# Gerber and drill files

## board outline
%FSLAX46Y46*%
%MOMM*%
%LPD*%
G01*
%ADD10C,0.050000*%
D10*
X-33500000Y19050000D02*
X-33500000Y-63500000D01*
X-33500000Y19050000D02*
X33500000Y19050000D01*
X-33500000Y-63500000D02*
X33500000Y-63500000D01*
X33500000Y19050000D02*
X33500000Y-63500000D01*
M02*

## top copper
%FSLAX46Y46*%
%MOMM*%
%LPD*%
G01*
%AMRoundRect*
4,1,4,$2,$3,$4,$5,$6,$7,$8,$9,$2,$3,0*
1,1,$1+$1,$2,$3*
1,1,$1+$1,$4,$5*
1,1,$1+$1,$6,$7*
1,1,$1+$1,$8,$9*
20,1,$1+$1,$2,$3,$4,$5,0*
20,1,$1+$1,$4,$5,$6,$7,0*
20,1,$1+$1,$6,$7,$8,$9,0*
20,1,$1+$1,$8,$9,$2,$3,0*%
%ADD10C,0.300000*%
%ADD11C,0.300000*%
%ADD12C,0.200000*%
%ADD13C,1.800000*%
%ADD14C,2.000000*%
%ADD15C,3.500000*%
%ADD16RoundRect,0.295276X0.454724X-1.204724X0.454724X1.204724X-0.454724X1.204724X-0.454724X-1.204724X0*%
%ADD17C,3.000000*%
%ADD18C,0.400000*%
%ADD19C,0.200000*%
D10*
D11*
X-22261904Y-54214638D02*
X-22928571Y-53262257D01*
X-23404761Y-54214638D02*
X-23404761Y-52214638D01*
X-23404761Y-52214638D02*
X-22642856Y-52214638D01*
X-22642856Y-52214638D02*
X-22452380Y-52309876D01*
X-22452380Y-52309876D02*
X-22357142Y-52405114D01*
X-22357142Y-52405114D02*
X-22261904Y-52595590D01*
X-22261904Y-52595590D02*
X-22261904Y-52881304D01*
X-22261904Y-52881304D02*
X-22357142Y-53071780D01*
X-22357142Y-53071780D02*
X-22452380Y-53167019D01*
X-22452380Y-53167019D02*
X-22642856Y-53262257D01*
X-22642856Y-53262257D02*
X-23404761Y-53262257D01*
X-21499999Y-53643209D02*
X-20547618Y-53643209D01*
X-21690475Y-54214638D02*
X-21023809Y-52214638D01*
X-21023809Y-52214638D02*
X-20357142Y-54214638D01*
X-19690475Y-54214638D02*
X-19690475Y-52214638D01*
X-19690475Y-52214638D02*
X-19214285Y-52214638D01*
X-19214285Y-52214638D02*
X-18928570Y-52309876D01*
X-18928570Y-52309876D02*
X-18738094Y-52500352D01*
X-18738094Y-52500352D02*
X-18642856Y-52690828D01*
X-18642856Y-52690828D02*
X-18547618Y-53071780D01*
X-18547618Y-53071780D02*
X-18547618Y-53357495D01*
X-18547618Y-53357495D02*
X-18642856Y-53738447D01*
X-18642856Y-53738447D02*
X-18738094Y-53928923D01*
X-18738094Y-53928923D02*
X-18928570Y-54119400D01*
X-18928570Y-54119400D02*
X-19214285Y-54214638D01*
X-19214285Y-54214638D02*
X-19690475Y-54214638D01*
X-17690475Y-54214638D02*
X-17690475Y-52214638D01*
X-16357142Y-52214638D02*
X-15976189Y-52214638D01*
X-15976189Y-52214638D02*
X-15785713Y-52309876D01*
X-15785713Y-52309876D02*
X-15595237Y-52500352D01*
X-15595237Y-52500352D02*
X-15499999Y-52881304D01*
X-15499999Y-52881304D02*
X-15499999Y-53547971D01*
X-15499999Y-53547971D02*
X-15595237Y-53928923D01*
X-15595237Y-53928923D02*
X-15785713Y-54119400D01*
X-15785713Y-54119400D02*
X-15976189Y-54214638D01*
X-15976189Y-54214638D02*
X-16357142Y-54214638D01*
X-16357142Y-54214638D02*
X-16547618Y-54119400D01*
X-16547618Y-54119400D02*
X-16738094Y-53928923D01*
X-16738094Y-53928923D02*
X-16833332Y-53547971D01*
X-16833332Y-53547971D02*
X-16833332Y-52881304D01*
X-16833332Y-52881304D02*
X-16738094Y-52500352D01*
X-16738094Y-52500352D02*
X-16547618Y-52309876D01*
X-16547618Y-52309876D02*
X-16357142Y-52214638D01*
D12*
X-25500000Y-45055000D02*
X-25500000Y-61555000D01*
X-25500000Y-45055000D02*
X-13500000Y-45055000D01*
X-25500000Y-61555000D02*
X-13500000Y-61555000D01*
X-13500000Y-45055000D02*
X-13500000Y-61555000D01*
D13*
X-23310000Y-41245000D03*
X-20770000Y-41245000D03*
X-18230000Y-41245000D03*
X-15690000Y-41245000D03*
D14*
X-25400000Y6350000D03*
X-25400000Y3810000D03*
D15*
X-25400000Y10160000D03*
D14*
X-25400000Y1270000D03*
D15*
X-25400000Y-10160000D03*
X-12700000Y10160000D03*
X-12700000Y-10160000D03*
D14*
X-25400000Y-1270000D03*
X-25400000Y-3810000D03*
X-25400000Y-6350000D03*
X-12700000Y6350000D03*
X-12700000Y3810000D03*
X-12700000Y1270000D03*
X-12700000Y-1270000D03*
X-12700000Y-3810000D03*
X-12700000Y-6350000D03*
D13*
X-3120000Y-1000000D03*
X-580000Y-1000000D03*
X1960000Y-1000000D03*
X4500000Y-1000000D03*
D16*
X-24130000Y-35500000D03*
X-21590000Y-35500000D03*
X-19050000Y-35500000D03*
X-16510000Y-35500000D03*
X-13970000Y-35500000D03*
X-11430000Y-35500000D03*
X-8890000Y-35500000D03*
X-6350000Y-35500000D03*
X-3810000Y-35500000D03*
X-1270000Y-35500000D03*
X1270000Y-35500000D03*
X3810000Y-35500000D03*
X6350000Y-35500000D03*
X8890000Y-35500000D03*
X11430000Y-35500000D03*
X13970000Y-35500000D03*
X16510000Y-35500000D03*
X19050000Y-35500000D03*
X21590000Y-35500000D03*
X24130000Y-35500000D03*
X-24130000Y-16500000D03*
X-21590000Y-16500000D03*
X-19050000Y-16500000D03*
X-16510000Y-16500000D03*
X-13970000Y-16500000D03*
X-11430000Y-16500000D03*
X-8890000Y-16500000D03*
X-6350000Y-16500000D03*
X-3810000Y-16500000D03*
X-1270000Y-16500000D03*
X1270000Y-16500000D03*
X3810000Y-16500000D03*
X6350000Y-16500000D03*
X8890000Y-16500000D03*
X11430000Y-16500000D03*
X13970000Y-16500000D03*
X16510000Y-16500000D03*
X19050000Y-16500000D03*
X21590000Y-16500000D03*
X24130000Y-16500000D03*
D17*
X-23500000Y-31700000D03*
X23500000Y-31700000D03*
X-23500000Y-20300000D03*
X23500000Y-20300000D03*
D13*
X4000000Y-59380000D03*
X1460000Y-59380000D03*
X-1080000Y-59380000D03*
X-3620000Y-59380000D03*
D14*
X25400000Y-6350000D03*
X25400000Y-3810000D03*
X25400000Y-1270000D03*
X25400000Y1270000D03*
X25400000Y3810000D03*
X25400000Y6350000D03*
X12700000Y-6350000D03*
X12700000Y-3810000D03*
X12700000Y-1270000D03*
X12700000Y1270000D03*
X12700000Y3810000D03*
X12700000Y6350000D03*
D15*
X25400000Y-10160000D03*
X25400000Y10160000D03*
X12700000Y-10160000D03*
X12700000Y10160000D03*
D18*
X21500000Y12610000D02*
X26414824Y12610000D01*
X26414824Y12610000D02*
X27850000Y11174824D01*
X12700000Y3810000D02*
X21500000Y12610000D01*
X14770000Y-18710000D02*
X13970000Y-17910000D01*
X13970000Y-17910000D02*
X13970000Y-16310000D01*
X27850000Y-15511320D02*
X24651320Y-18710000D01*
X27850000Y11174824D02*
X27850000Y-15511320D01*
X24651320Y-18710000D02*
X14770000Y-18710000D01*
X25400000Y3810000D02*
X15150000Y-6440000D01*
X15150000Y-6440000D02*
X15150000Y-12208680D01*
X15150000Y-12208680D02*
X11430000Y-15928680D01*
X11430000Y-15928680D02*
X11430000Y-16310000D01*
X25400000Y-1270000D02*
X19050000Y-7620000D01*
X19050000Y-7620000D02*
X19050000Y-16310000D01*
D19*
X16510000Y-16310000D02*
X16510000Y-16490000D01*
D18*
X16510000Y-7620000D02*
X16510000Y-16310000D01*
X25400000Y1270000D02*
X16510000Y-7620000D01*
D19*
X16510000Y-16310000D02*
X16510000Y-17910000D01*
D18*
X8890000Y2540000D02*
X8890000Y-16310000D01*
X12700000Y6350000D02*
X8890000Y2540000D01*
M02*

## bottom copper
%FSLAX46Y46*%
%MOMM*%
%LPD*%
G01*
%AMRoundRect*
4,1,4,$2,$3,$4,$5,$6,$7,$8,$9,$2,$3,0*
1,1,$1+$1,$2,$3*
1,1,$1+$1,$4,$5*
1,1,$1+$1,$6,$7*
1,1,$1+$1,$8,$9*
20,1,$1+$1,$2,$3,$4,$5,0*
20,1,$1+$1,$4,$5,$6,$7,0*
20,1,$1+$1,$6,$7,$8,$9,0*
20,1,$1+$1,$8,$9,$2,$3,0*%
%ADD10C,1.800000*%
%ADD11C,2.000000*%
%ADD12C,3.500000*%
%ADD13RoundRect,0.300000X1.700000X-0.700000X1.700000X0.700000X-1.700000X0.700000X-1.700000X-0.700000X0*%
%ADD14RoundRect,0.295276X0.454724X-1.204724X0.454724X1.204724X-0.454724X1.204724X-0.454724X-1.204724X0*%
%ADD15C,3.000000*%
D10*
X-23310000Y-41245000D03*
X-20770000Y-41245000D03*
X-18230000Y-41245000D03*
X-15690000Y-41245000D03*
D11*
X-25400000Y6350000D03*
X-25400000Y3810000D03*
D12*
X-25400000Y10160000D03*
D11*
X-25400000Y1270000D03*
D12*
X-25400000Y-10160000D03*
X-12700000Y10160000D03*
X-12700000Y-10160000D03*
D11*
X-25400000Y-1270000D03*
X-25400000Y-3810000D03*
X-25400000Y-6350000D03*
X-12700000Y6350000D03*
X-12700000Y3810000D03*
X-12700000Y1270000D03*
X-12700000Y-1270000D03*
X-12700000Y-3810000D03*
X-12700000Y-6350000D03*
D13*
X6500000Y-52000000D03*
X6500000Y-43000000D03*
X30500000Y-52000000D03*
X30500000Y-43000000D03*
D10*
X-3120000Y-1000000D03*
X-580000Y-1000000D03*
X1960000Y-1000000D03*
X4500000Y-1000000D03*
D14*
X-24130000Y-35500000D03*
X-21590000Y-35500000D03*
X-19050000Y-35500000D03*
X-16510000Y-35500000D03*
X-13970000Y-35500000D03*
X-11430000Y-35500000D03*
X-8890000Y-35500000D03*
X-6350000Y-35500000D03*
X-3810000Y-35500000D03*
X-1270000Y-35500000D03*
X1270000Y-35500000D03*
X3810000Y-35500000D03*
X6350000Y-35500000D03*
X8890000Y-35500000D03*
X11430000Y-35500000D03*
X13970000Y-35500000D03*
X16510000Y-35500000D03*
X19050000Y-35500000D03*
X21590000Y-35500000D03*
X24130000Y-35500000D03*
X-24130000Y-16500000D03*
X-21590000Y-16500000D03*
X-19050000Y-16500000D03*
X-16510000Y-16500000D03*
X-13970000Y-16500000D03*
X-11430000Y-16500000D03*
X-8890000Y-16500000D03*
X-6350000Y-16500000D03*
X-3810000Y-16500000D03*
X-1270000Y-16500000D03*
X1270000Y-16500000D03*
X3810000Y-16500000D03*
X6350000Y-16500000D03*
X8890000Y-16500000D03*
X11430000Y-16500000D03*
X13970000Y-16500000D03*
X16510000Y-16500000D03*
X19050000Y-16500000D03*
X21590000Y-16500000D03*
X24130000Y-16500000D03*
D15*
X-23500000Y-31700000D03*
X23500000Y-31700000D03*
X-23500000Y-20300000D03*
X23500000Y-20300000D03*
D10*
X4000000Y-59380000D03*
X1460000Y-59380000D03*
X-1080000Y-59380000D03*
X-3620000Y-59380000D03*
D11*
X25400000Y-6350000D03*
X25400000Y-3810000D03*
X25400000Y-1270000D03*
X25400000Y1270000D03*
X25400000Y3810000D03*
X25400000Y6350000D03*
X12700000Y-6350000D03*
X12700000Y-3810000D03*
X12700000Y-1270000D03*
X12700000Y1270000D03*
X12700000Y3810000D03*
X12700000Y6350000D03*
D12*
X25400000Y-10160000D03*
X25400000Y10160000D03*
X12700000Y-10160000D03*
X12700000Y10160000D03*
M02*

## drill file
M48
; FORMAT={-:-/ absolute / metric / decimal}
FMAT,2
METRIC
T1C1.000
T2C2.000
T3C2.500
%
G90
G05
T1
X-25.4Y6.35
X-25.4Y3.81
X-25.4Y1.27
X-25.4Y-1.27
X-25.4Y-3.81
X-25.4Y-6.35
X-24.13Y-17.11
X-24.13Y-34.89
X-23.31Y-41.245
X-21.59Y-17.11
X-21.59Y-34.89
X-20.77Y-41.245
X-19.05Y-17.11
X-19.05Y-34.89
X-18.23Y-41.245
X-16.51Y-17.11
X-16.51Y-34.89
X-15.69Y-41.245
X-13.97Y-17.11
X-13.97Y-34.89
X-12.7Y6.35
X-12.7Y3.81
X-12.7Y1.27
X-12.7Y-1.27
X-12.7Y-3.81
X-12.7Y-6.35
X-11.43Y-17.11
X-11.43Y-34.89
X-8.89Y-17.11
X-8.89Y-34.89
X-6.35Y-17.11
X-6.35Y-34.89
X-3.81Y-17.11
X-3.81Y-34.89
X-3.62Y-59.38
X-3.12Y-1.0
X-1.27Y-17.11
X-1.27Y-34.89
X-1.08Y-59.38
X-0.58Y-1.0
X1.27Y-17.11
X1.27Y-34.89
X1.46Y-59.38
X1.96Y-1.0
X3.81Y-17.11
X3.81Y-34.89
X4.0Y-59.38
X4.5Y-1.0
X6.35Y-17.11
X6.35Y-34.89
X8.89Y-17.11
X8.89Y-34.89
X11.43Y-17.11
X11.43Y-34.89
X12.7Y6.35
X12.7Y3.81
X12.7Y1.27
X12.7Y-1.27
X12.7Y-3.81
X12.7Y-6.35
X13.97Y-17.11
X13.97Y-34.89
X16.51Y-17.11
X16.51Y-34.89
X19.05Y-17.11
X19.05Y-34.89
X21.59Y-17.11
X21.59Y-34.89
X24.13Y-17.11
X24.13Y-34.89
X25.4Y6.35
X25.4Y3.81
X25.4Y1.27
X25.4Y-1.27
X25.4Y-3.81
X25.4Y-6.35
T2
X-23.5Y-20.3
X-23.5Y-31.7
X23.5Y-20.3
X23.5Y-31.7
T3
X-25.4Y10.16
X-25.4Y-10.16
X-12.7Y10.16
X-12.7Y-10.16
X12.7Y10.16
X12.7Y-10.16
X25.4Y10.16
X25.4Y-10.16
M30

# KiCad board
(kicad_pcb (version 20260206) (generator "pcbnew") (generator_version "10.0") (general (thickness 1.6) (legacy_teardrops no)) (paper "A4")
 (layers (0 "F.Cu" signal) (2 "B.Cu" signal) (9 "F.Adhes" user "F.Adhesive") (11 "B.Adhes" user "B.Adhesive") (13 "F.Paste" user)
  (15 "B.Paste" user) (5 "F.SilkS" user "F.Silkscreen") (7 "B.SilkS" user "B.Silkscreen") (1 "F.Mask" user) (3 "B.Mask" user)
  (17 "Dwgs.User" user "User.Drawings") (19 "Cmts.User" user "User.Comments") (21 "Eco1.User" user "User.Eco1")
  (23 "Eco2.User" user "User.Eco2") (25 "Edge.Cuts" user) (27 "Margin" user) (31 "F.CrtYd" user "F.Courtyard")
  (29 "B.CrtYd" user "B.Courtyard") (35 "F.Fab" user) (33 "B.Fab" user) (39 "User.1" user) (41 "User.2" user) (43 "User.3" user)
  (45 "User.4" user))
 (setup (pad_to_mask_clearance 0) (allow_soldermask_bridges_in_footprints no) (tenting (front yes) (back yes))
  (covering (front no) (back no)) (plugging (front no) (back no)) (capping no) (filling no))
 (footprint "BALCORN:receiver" (layer "F.Cu") (at -19.5 53.305)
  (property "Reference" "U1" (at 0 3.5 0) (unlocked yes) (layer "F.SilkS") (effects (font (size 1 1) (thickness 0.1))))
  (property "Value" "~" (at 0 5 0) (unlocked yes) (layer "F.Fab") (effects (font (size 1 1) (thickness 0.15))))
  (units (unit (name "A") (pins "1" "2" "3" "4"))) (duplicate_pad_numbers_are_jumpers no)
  (fp_line (start -6 -8.25) (end -6 8.25) (stroke (width 0.2) (type default)) (layer "F.Cu"))
  (fp_line (start -6 -8.25) (end 6 -8.25) (stroke (width 0.2) (type default)) (layer "F.Cu"))
  (fp_line (start -6 8.25) (end 6 8.25) (stroke (width 0.2) (type default)) (layer "F.Cu"))
  (fp_line (start 6 -8.25) (end 6 8.25) (stroke (width 0.2) (type default)) (layer "F.Cu"))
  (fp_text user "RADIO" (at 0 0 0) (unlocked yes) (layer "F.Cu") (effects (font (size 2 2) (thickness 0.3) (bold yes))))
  (pad "1" thru_hole circle (at -3.81 -12.06) (size 1.8 1.8) (drill 1) (layers "*.Cu" "*.Mask") (remove_unused_layers no)
   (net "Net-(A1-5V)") (thermal_bridge_angle 90))
  (pad "2" thru_hole circle (at -1.27 -12.06) (size 1.8 1.8) (drill 1) (layers "*.Cu" "*.Mask") (remove_unused_layers no)
   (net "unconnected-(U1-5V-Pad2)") (thermal_bridge_angle 90))
  (pad "3" thru_hole circle (at 1.27 -12.06) (size 1.8 1.8) (drill 1) (layers "*.Cu" "*.Mask") (remove_unused_layers no)
   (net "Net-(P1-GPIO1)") (thermal_bridge_angle 90))
  (pad "4" thru_hole circle (at 3.81 -12.06) (size 1.8 1.8) (drill 1) (layers "*.Cu" "*.Mask") (remove_unused_layers no)
   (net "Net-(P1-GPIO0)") (thermal_bridge_angle 90)))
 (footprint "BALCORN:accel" (layer "F.Cu") (at -19.05 0)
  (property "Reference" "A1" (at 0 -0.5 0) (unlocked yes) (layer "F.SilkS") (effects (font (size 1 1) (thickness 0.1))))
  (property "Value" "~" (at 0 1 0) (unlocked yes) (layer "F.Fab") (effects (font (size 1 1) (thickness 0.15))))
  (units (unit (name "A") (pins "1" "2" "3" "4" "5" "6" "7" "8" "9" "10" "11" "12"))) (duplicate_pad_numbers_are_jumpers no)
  (pad "1" thru_hole circle (at -6.35 -6.35) (size 2 2) (drill 1) (layers "*.Cu" "*.Mask") (remove_unused_layers no) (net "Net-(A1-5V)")
   (thermal_bridge_angle 90))
  (pad "2" thru_hole circle (at -6.35 -3.81) (size 2 2) (drill 1) (layers "*.Cu" "*.Mask") (remove_unused_layers no)
   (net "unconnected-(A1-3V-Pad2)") (thermal_bridge_angle 90))
  (pad "3" thru_hole circle (at -6.35 -10.16) (size 3.5 3.5) (drill 2.5) (layers "*.Cu" "*.Mask") (remove_unused_layers no)
   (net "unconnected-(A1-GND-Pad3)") (thermal_bridge_angle 90))
  (pad "3" thru_hole circle (at -6.35 -1.27) (size 2 2) (drill 1) (layers "*.Cu" "*.Mask") (remove_unused_layers no)
   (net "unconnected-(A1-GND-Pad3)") (thermal_bridge_angle 90))
  (pad "3" thru_hole circle (at -6.35 10.16) (size 3.5 3.5) (drill 2.5) (layers "*.Cu" "*.Mask") (remove_unused_layers no)
   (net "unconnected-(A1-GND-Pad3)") (thermal_bridge_angle 90))
  (pad "3" thru_hole circle (at 6.35 -10.16) (size 3.5 3.5) (drill 2.5) (layers "*.Cu" "*.Mask") (remove_unused_layers no)
   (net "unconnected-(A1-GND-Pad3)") (thermal_bridge_angle 90))
  (pad "3" thru_hole circle (at 6.35 10.16) (size 3.5 3.5) (drill 2.5) (layers "*.Cu" "*.Mask") (remove_unused_layers no)
   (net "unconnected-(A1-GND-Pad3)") (thermal_bridge_angle 90))
  (pad "4" thru_hole circle (at -6.35 1.27) (size 2 2) (drill 1) (layers "*.Cu" "*.Mask") (remove_unused_layers no) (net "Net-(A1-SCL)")
   (thermal_bridge_angle 90))
  (pad "5" thru_hole circle (at -6.35 3.81) (size 2 2) (drill 1) (layers "*.Cu" "*.Mask") (remove_unused_layers no) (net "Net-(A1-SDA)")
   (thermal_bridge_angle 90))
  (pad "6" thru_hole circle (at -6.35 6.35) (size 2 2) (drill 1) (layers "*.Cu" "*.Mask") (remove_unused_layers no)
   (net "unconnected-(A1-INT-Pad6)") (thermal_bridge_angle 90))
  (pad "7" thru_hole circle (at 6.35 -6.35) (size 2 2) (drill 1) (layers "*.Cu" "*.Mask") (remove_unused_layers no)
   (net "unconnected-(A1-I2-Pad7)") (thermal_bridge_angle 90))
  (pad "8" thru_hole circle (at 6.35 -3.81) (size 2 2) (drill 1) (layers "*.Cu" "*.Mask") (remove_unused_layers no)
   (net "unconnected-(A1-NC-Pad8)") (thermal_bridge_angle 90))
  (pad "9" thru_hole circle (at 6.35 -1.27) (size 2 2) (drill 1) (layers "*.Cu" "*.Mask") (remove_unused_layers no)
   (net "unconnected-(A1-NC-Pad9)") (thermal_bridge_angle 90))
  (pad "10" thru_hole circle (at 6.35 1.27) (size 2 2) (drill 1) (layers "*.Cu" "*.Mask") (remove_unused_layers no)
   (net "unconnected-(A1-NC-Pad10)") (thermal_bridge_angle 90))
  (pad "11" thru_hole circle (at 6.35 3.81) (size 2 2) (drill 1) (layers "*.Cu" "*.Mask") (remove_unused_layers no) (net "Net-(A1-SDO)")
   (thermal_bridge_angle 90))
  (pad "12" thru_hole circle (at 6.35 6.35) (size 2 2) (drill 1) (layers "*.Cu" "*.Mask") (remove_unused_layers no) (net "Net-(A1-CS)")
   (thermal_bridge_angle 90)))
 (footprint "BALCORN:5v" (layer "F.Cu") (at 18.5 47.5 90)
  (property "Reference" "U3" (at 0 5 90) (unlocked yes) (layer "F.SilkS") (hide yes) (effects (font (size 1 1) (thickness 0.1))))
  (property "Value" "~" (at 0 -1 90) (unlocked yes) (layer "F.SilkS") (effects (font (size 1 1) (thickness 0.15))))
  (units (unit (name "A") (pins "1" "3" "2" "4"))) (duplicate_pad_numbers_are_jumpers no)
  (pad "1" smd roundrect (at -4.5 -12 90) (size 2 4) (layers "*.Mask" "B.Cu") (roundrect_rratio 0.15) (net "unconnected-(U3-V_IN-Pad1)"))
  (pad "2" smd roundrect (at 4.5 -12 90) (size 2 4) (layers "*.Mask" "B.Cu") (roundrect_rratio 0.15) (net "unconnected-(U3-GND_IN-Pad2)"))
  (pad "3" smd roundrect (at -4.5 12 90) (size 2 4) (layers "*.Mask" "B.Cu") (roundrect_rratio 0.15) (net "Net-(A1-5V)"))
  (pad "4" smd roundrect (at 4.5 12 90) (size 2 4) (layers "*.Mask" "B.Cu") (roundrect_rratio 0.15) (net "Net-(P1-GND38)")))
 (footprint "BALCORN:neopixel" (layer "F.Cu") (at 0.69 1)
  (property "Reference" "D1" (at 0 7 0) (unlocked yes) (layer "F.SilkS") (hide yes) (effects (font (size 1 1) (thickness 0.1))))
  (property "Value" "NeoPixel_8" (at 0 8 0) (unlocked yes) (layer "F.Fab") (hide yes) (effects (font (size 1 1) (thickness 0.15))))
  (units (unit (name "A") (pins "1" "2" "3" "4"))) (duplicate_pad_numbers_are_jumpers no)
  (pad "1" thru_hole circle (at -3.81 0) (size 1.8 1.8) (drill 1) (layers "*.Cu" "*.Mask") (remove_unused_layers no) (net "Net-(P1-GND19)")
   (thermal_bridge_angle 90))
  (pad "2" thru_hole circle (at -1.27 0) (size 1.8 1.8) (drill 1) (layers "*.Cu" "*.Mask") (remove_unused_layers no) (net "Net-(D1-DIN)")
   (thermal_bridge_angle 90))
  (pad "3" thru_hole circle (at 1.27 0) (size 1.8 1.8) (drill 1) (layers "*.Cu" "*.Mask") (remove_unused_layers no) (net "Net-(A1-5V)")
   (thermal_bridge_angle 90))
  (pad "4" thru_hole circle (at 3.81 0) (size 1.8 1.8) (drill 1) (layers "*.Cu" "*.Mask") (remove_unused_layers no) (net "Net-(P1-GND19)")
   (thermal_bridge_angle 90)))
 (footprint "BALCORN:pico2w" (layer "F.Cu") (at 0 26 90)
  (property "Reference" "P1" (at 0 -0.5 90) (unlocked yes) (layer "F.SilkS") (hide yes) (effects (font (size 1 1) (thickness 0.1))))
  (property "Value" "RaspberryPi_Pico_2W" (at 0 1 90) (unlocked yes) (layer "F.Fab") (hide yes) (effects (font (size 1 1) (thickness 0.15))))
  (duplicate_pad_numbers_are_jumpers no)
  (pad "1" thru_hole roundrect (at -8.89 -24.13 90) (size 3 1.5) (drill 1 (offset -0.61 0)) (layers "*.Cu" "*.Mask")
   (remove_unused_layers no) (roundrect_rratio 0.1968503937) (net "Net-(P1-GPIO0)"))
  (pad "2" thru_hole roundrect (at -8.89 -21.59 90) (size 3 1.5) (drill 1 (offset -0.61 0)) (layers "*.Cu" "*.Mask")
   (remove_unused_layers no) (roundrect_rratio 0.1968503937) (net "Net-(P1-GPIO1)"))
  (pad "3" thru_hole roundrect (at -8.89 -19.05 90) (size 3 1.5) (drill 1 (offset -0.61 0)) (layers "*.Cu" "*.Mask")
   (remove_unused_layers no) (roundrect_rratio 0.1968503937) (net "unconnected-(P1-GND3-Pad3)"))
  (pad "4" thru_hole roundrect (at -8.89 -16.51 90) (size 3 1.5) (drill 1 (offset -0.61 0)) (layers "*.Cu" "*.Mask")
   (remove_unused_layers no) (roundrect_rratio 0.1968503937) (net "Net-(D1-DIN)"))
  (pad "5" thru_hole roundrect (at -8.89 -13.97 90) (size 3 1.5) (drill 1 (offset -0.61 0)) (layers "*.Cu" "*.Mask")
   (remove_unused_layers no) (roundrect_rratio 0.1968503937) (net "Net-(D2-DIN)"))
  (pad "6" thru_hole roundrect (at -8.89 -11.43 90) (size 3 1.5) (drill 1 (offset -0.61 0)) (layers "*.Cu" "*.Mask")
   (remove_unused_layers no) (roundrect_rratio 0.1968503937) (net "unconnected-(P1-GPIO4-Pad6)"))
  (pad "7" thru_hole roundrect (at -8.89 -8.89 90) (size 3 1.5) (drill 1 (offset -0.61 0)) (layers "*.Cu" "*.Mask")
   (remove_unused_layers no) (roundrect_rratio 0.1968503937) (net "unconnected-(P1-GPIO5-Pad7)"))
  (pad "8" thru_hole roundrect (at -8.89 -6.35 90) (size 3 1.5) (drill 1 (offset -0.61 0)) (layers "*.Cu" "*.Mask")
   (remove_unused_layers no) (roundrect_rratio 0.1968503937) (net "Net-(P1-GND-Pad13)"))
  (pad "9" thru_hole roundrect (at -8.89 -3.81 90) (size 3 1.5) (drill 1 (offset -0.61 0)) (layers "*.Cu" "*.Mask")
   (remove_unused_layers no) (roundrect_rratio 0.1968503937) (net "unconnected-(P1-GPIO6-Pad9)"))
  (pad "10" thru_hole roundrect (at -8.89 -1.27 90) (size 3 1.5) (drill 1 (offset -0.61 0)) (layers "*.Cu" "*.Mask")
   (remove_unused_layers no) (roundrect_rratio 0.1968503937) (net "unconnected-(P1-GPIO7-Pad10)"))
  (pad "11" thru_hole roundrect (at -8.89 1.27 90) (size 3 1.5) (drill 1 (offset -0.61 0)) (layers "*.Cu" "*.Mask")
   (remove_unused_layers no) (roundrect_rratio 0.1968503937) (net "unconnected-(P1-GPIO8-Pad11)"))
  (pad "12" thru_hole roundrect (at -8.89 3.81 90) (size 3 1.5) (drill 1 (offset -0.61 0)) (layers "*.Cu" "*.Mask")
   (remove_unused_layers no) (roundrect_rratio 0.1968503937) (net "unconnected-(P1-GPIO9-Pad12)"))
  (pad "13" thru_hole roundrect (at -8.89 6.35 90) (size 3 1.5) (drill 1 (offset -0.61 0)) (layers "*.Cu" "*.Mask")
   (remove_unused_layers no) (roundrect_rratio 0.1968503937) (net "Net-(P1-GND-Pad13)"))
  (pad "14" thru_hole roundrect (at -8.89 8.89 90) (size 3 1.5) (drill 1 (offset -0.61 0)) (layers "*.Cu" "*.Mask")
   (remove_unused_layers no) (roundrect_rratio 0.1968503937) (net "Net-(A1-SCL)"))
  (pad "15" thru_hole roundrect (at -8.89 11.43 90) (size 3 1.5) (drill 1 (offset -0.61 0)) (layers "*.Cu" "*.Mask")
   (remove_unused_layers no) (roundrect_rratio 0.1968503937) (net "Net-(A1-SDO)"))
  (pad "16" thru_hole roundrect (at -8.89 13.97 90) (size 3 1.5) (drill 1 (offset -0.61 0)) (layers "*.Cu" "*.Mask")
   (remove_unused_layers no) (roundrect_rratio 0.1968503937) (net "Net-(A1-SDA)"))
  (pad "17" thru_hole roundrect (at -8.89 16.51 90) (size 3 1.5) (drill 1 (offset -0.61 0)) (layers "*.Cu" "*.Mask")
   (remove_unused_layers no) (roundrect_rratio 0.1968503937) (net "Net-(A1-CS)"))
  (pad "18" thru_hole roundrect (at -8.89 19.05 90) (size 3 1.5) (drill 1 (offset -0.61 0)) (layers "*.Cu" "*.Mask")
   (remove_unused_layers no) (roundrect_rratio 0.1968503937) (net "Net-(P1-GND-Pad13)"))
  (pad "19" thru_hole roundrect (at -8.89 21.59 90) (size 3 1.5) (drill 1 (offset -0.61 0)) (layers "*.Cu" "*.Mask")
   (remove_unused_layers no) (roundrect_rratio 0.1968503937) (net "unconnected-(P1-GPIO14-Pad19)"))
  (pad "20" thru_hole roundrect (at -8.89 24.13 90) (size 3 1.5) (drill 1 (offset -0.61 0)) (layers "*.Cu" "*.Mask")
   (remove_unused_layers no) (roundrect_rratio 0.1968503937) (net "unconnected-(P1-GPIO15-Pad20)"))
  (pad "21" thru_hole roundrect (at 8.89 -24.13 90) (size 3 1.5) (drill 1 (offset 0.61 0)) (layers "*.Cu" "*.Mask")
   (remove_unused_layers no) (roundrect_rratio 0.1968503937) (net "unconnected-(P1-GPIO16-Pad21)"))
  (pad "22" thru_hole roundrect (at 8.89 -21.59 90) (size 3 1.5) (drill 1 (offset 0.61 0)) (layers "*.Cu" "*.Mask")
   (remove_unused_layers no) (roundrect_rratio 0.1968503937) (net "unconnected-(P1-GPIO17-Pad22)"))
  (pad "23" thru_hole roundrect (at 8.89 -19.05 90) (size 3 1.5) (drill 1 (offset 0.61 0)) (layers "*.Cu" "*.Mask")
   (remove_unused_layers no) (roundrect_rratio 0.1968503937) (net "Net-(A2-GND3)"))
  (pad "24" thru_hole roundrect (at 8.89 -16.51 90) (size 3 1.5) (drill 1 (offset 0.61 0)) (layers "*.Cu" "*.Mask")
   (remove_unused_layers no) (roundrect_rratio 0.1968503937) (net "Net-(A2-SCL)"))
  (pad "25" thru_hole roundrect (at 8.89 -13.97 90) (size 3 1.5) (drill 1 (offset 0.61 0)) (layers "*.Cu" "*.Mask")
   (remove_unused_layers no) (roundrect_rratio 0.1968503937) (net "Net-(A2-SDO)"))
  (pad "26" thru_hole roundrect (at 8.89 -11.43 90) (size 3 1.5) (drill 1 (offset 0.61 0)) (layers "*.Cu" "*.Mask")
   (remove_unused_layers no) (roundrect_rratio 0.1968503937) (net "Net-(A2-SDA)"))
  (pad "27" thru_hole roundrect (at 8.89 -8.89 90) (size 3 1.5) (drill 1 (offset 0.61 0)) (layers "*.Cu" "*.Mask") (remove_unused_layers no)
   (roundrect_rratio 0.1968503937) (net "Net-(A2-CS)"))
  (pad "28" thru_hole roundrect (at 8.89 -6.35 90) (size 3 1.5) (drill 1 (offset 0.61 0)) (layers "*.Cu" "*.Mask") (remove_unused_layers no)
   (roundrect_rratio 0.1968503937) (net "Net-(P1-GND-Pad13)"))
  (pad "29" thru_hole roundrect (at 8.89 -3.81 90) (size 3 1.5) (drill 1 (offset 0.61 0)) (layers "*.Cu" "*.Mask") (remove_unused_layers no)
   (roundrect_rratio 0.1968503937) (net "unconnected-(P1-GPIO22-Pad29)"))
  (pad "30" thru_hole roundrect (at 8.89 -1.27 90) (size 3 1.5) (drill 1 (offset 0.61 0)) (layers "*.Cu" "*.Mask") (remove_unused_layers no)
   (roundrect_rratio 0.1968503937) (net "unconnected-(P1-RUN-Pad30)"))
  (pad "31" thru_hole roundrect (at 8.89 1.27 90) (size 3 1.5) (drill 1 (offset 0.61 0)) (layers "*.Cu" "*.Mask") (remove_unused_layers no)
   (roundrect_rratio 0.1968503937) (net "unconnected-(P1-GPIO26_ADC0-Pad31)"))
  (pad "32" thru_hole roundrect (at 8.89 3.81 90) (size 3 1.5) (drill 1 (offset 0.61 0)) (layers "*.Cu" "*.Mask") (remove_unused_layers no)
   (roundrect_rratio 0.1968503937) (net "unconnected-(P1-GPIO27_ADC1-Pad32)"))
  (pad "33" thru_hole roundrect (at 8.89 6.35 90) (size 3 1.5) (drill 1 (offset 0.61 0)) (layers "*.Cu" "*.Mask") (remove_unused_layers no)
   (roundrect_rratio 0.1968503937) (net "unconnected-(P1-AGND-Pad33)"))
  (pad "34" thru_hole roundrect (at 8.89 8.89 90) (size 3 1.5) (drill 1 (offset 0.61 0)) (layers "*.Cu" "*.Mask") (remove_unused_layers no)
   (roundrect_rratio 0.1968503937) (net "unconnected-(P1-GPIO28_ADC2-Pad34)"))
  (pad "35" thru_hole roundrect (at 8.89 11.43 90) (size 3 1.5) (drill 1 (offset 0.61 0)) (layers "*.Cu" "*.Mask") (remove_unused_layers no)
   (roundrect_rratio 0.1968503937) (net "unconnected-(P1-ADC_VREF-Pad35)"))
  (pad "36" thru_hole roundrect (at 8.89 13.97 90) (size 3 1.5) (drill 1 (offset 0.61 0)) (layers "*.Cu" "*.Mask") (remove_unused_layers no)
   (roundrect_rratio 0.1968503937) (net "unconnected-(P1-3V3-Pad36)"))
  (pad "37" thru_hole roundrect (at 8.89 16.51 90) (size 3 1.5) (drill 1 (offset 0.61 0)) (layers "*.Cu" "*.Mask") (remove_unused_layers no)
   (roundrect_rratio 0.1968503937) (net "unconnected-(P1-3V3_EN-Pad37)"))
  (pad "38" thru_hole roundrect (at 8.89 19.05 90) (size 3 1.5) (drill 1 (offset 0.61 0)) (layers "*.Cu" "*.Mask") (remove_unused_layers no)
   (roundrect_rratio 0.1968503937) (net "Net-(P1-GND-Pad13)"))
  (pad "39" thru_hole roundrect (at 8.89 21.59 90) (size 3 1.5) (drill 1 (offset 0.61 0)) (layers "*.Cu" "*.Mask") (remove_unused_layers no)
   (roundrect_rratio 0.1968503937) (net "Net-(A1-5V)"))
  (pad "40" thru_hole roundrect (at 8.89 24.13 90) (size 3 1.5) (drill 1 (offset 0.61 0)) (layers "*.Cu" "*.Mask") (remove_unused_layers no)
   (roundrect_rratio 0.1968503937) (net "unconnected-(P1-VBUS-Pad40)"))
  (pad "41" thru_hole circle (at -5.7 -23.5 90) (size 3 3) (drill 2) (layers "*.Cu" "*.Mask") (remove_unused_layers no)
   (thermal_bridge_angle 90))
  (pad "41" thru_hole circle (at -5.7 23.5 90) (size 3 3) (drill 2) (layers "*.Cu" "*.Mask") (remove_unused_layers no)
   (thermal_bridge_angle 90))
  (pad "41" thru_hole circle (at 5.7 -23.5 90) (size 3 3) (drill 2) (layers "*.Cu" "*.Mask") (remove_unused_layers no)
   (thermal_bridge_angle 90))
  (pad "41" thru_hole circle (at 5.7 23.5 90) (size 3 3) (drill 2) (layers "*.Cu" "*.Mask") (remove_unused_layers no)
   (thermal_bridge_angle 90)))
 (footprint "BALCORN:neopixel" (layer "F.Cu") (at 0.19 59.38 180)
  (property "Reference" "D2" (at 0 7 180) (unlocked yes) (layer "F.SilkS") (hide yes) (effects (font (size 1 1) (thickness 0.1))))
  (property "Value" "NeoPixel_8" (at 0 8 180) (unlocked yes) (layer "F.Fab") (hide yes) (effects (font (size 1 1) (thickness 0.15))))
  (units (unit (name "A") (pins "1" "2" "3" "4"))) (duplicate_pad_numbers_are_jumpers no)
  (pad "1" thru_hole circle (at -3.81 0 180) (size 1.8 1.8) (drill 1) (layers "*.Cu" "*.Mask") (remove_unused_layers no)
   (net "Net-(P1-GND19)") (thermal_bridge_angle 90))
  (pad "2" thru_hole circle (at -1.27 0 180) (size 1.8 1.8) (drill 1) (layers "*.Cu" "*.Mask") (remove_unused_layers no)
   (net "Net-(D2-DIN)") (thermal_bridge_angle 90))
  (pad "3" thru_hole circle (at 1.27 0 180) (size 1.8 1.8) (drill 1) (layers "*.Cu" "*.Mask") (remove_unused_layers no) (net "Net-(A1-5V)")
   (thermal_bridge_angle 90))
  (pad "4" thru_hole circle (at 3.81 0 180) (size 1.8 1.8) (drill 1) (layers "*.Cu" "*.Mask") (remove_unused_layers no)
   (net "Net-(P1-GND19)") (thermal_bridge_angle 90)))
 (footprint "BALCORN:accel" (layer "F.Cu") (at 19.05 0 180)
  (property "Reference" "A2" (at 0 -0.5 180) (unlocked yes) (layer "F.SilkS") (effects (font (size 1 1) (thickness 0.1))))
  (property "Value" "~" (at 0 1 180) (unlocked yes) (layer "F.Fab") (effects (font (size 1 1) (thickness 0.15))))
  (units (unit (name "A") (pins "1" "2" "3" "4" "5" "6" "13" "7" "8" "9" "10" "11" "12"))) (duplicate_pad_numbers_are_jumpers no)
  (pad "1" thru_hole circle (at -6.35 -6.35 180) (size 2 2) (drill 1) (layers "*.Cu" "*.Mask") (remove_unused_layers no) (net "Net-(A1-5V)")
   (thermal_bridge_angle 90))
  (pad "2" thru_hole circle (at -6.35 -3.81 180) (size 2 2) (drill 1) (layers "*.Cu" "*.Mask") (remove_unused_layers no)
   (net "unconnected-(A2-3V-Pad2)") (thermal_bridge_angle 90))
  (pad "3" thru_hole circle (at -6.35 -1.27 180) (size 2 2) (drill 1) (layers "*.Cu" "*.Mask") (remove_unused_layers no)
   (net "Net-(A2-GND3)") (thermal_bridge_angle 90))
  (pad "4" thru_hole circle (at -6.35 1.27 180) (size 2 2) (drill 1) (layers "*.Cu" "*.Mask") (remove_unused_layers no) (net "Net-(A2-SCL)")
   (thermal_bridge_angle 90))
  (pad "5" thru_hole circle (at -6.35 3.81 180) (size 2 2) (drill 1) (layers "*.Cu" "*.Mask") (remove_unused_layers no) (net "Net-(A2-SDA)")
   (thermal_bridge_angle 90))
  (pad "6" thru_hole circle (at -6.35 6.35 180) (size 2 2) (drill 1) (layers "*.Cu" "*.Mask") (remove_unused_layers no)
   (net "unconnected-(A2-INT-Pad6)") (thermal_bridge_angle 90))
  (pad "7" thru_hole circle (at 6.35 -6.35 180) (size 2 2) (drill 1) (layers "*.Cu" "*.Mask") (remove_unused_layers no)
   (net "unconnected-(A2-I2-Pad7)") (thermal_bridge_angle 90))
  (pad "8" thru_hole circle (at 6.35 -3.81 180) (size 2 2) (drill 1) (layers "*.Cu" "*.Mask") (remove_unused_layers no)
   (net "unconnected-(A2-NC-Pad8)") (thermal_bridge_angle 90))
  (pad "9" thru_hole circle (at 6.35 -1.27 180) (size 2 2) (drill 1) (layers "*.Cu" "*.Mask") (remove_unused_layers no)
   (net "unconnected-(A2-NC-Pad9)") (thermal_bridge_angle 90))
  (pad "10" thru_hole circle (at 6.35 1.27 180) (size 2 2) (drill 1) (layers "*.Cu" "*.Mask") (remove_unused_layers no)
   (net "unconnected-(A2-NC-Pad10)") (thermal_bridge_angle 90))
  (pad "11" thru_hole circle (at 6.35 3.81 180) (size 2 2) (drill 1) (layers "*.Cu" "*.Mask") (remove_unused_layers no) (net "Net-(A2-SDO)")
   (thermal_bridge_angle 90))
  (pad "12" thru_hole circle (at 6.35 6.35 180) (size 2 2) (drill 1) (layers "*.Cu" "*.Mask") (remove_unused_layers no) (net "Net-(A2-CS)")
   (thermal_bridge_angle 90))
  (pad "13" thru_hole circle (at -6.35 -10.16 180) (size 3.5 3.5) (drill 2.5) (layers "*.Cu" "*.Mask") (remove_unused_layers no)
   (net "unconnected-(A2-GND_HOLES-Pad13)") (thermal_bridge_angle 90))
  (pad "13" thru_hole circle (at -6.35 10.16 180) (size 3.5 3.5) (drill 2.5) (layers "*.Cu" "*.Mask") (remove_unused_layers no)
   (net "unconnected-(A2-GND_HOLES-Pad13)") (thermal_bridge_angle 90))
  (pad "13" thru_hole circle (at 6.35 -10.16 180) (size 3.5 3.5) (drill 2.5) (layers "*.Cu" "*.Mask") (remove_unused_layers no)
   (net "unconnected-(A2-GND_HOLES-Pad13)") (thermal_bridge_angle 90))
  (pad "13" thru_hole circle (at 6.35 10.16 180) (size 3.5 3.5) (drill 2.5) (layers "*.Cu" "*.Mask") (remove_unused_layers no)
   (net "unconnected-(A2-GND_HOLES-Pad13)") (thermal_bridge_angle 90)))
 (gr_line (start -33.5 -19.05) (end -33.5 63.5) (stroke (width 0.05) (type default)) (layer "Edge.Cuts"))
 (gr_line (start -33.5 -19.05) (end 33.5 -19.05) (stroke (width 0.05) (type default)) (layer "Edge.Cuts"))
 (gr_line (start -33.5 63.5) (end 33.5 63.5) (stroke (width 0.05) (type default)) (layer "Edge.Cuts"))
 (gr_line (start 33.5 -19.05) (end 33.5 63.5) (stroke (width 0.05) (type default)) (layer "Edge.Cuts"))
 (segment (start 21.5 -12.61) (end 26.414824 -12.61) (width 0.4) (layer "F.Cu") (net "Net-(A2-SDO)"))
 (segment (start 26.414824 -12.61) (end 27.85 -11.174824) (width 0.4) (layer "F.Cu") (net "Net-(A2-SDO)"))
 (segment (start 12.7 -3.81) (end 21.5 -12.61) (width 0.4) (layer "F.Cu") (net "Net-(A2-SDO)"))
 (segment (start 14.77 18.71) (end 13.97 17.91) (width 0.4) (layer "F.Cu") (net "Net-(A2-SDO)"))
 (segment (start 13.97 17.91) (end 13.97 16.31) (width 0.4) (layer "F.Cu") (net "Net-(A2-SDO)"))
 (segment (start 27.85 15.51132) (end 24.65132 18.71) (width 0.4) (layer "F.Cu") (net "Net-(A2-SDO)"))
 (segment (start 27.85 -11.174824) (end 27.85 15.51132) (width 0.4) (layer "F.Cu") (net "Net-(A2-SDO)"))
 (segment (start 24.65132 18.71) (end 14.77 18.71) (width 0.4) (layer "F.Cu") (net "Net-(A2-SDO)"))
 (segment (start 25.4 -3.81) (end 15.15 6.44) (width 0.4) (layer "F.Cu") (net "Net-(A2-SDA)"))
 (segment (start 15.15 6.44) (end 15.15 12.20868) (width 0.4) (layer "F.Cu") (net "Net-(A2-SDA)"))
 (segment (start 15.15 12.20868) (end 11.43 15.92868) (width 0.4) (layer "F.Cu") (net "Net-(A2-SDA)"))
 (segment (start 11.43 15.92868) (end 11.43 16.31) (width 0.4) (layer "F.Cu") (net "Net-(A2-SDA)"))
 (segment (start 25.4 1.27) (end 19.05 7.62) (width 0.4) (layer "F.Cu") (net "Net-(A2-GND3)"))
 (segment (start 19.05 7.62) (end 19.05 16.31) (width 0.4) (layer "F.Cu") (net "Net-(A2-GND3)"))
 (segment (start 16.51 16.31) (end 16.51 16.49) (width 0.2) (layer "F.Cu") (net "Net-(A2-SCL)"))
 (segment (start 16.51 7.62) (end 16.51 16.31) (width 0.4) (layer "F.Cu") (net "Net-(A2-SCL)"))
 (segment (start 25.4 -1.27) (end 16.51 7.62) (width 0.4) (layer "F.Cu") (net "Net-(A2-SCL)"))
 (segment (start 16.51 16.31) (end 16.51 17.91) (width 0.2) (layer "F.Cu") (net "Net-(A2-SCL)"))
 (segment (start 8.89 -2.54) (end 8.89 16.31) (width 0.4) (layer "F.Cu") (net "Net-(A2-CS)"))
 (segment (start 12.7 -6.35) (end 8.89 -2.54) (width 0.4) (layer "F.Cu") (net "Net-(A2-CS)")))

